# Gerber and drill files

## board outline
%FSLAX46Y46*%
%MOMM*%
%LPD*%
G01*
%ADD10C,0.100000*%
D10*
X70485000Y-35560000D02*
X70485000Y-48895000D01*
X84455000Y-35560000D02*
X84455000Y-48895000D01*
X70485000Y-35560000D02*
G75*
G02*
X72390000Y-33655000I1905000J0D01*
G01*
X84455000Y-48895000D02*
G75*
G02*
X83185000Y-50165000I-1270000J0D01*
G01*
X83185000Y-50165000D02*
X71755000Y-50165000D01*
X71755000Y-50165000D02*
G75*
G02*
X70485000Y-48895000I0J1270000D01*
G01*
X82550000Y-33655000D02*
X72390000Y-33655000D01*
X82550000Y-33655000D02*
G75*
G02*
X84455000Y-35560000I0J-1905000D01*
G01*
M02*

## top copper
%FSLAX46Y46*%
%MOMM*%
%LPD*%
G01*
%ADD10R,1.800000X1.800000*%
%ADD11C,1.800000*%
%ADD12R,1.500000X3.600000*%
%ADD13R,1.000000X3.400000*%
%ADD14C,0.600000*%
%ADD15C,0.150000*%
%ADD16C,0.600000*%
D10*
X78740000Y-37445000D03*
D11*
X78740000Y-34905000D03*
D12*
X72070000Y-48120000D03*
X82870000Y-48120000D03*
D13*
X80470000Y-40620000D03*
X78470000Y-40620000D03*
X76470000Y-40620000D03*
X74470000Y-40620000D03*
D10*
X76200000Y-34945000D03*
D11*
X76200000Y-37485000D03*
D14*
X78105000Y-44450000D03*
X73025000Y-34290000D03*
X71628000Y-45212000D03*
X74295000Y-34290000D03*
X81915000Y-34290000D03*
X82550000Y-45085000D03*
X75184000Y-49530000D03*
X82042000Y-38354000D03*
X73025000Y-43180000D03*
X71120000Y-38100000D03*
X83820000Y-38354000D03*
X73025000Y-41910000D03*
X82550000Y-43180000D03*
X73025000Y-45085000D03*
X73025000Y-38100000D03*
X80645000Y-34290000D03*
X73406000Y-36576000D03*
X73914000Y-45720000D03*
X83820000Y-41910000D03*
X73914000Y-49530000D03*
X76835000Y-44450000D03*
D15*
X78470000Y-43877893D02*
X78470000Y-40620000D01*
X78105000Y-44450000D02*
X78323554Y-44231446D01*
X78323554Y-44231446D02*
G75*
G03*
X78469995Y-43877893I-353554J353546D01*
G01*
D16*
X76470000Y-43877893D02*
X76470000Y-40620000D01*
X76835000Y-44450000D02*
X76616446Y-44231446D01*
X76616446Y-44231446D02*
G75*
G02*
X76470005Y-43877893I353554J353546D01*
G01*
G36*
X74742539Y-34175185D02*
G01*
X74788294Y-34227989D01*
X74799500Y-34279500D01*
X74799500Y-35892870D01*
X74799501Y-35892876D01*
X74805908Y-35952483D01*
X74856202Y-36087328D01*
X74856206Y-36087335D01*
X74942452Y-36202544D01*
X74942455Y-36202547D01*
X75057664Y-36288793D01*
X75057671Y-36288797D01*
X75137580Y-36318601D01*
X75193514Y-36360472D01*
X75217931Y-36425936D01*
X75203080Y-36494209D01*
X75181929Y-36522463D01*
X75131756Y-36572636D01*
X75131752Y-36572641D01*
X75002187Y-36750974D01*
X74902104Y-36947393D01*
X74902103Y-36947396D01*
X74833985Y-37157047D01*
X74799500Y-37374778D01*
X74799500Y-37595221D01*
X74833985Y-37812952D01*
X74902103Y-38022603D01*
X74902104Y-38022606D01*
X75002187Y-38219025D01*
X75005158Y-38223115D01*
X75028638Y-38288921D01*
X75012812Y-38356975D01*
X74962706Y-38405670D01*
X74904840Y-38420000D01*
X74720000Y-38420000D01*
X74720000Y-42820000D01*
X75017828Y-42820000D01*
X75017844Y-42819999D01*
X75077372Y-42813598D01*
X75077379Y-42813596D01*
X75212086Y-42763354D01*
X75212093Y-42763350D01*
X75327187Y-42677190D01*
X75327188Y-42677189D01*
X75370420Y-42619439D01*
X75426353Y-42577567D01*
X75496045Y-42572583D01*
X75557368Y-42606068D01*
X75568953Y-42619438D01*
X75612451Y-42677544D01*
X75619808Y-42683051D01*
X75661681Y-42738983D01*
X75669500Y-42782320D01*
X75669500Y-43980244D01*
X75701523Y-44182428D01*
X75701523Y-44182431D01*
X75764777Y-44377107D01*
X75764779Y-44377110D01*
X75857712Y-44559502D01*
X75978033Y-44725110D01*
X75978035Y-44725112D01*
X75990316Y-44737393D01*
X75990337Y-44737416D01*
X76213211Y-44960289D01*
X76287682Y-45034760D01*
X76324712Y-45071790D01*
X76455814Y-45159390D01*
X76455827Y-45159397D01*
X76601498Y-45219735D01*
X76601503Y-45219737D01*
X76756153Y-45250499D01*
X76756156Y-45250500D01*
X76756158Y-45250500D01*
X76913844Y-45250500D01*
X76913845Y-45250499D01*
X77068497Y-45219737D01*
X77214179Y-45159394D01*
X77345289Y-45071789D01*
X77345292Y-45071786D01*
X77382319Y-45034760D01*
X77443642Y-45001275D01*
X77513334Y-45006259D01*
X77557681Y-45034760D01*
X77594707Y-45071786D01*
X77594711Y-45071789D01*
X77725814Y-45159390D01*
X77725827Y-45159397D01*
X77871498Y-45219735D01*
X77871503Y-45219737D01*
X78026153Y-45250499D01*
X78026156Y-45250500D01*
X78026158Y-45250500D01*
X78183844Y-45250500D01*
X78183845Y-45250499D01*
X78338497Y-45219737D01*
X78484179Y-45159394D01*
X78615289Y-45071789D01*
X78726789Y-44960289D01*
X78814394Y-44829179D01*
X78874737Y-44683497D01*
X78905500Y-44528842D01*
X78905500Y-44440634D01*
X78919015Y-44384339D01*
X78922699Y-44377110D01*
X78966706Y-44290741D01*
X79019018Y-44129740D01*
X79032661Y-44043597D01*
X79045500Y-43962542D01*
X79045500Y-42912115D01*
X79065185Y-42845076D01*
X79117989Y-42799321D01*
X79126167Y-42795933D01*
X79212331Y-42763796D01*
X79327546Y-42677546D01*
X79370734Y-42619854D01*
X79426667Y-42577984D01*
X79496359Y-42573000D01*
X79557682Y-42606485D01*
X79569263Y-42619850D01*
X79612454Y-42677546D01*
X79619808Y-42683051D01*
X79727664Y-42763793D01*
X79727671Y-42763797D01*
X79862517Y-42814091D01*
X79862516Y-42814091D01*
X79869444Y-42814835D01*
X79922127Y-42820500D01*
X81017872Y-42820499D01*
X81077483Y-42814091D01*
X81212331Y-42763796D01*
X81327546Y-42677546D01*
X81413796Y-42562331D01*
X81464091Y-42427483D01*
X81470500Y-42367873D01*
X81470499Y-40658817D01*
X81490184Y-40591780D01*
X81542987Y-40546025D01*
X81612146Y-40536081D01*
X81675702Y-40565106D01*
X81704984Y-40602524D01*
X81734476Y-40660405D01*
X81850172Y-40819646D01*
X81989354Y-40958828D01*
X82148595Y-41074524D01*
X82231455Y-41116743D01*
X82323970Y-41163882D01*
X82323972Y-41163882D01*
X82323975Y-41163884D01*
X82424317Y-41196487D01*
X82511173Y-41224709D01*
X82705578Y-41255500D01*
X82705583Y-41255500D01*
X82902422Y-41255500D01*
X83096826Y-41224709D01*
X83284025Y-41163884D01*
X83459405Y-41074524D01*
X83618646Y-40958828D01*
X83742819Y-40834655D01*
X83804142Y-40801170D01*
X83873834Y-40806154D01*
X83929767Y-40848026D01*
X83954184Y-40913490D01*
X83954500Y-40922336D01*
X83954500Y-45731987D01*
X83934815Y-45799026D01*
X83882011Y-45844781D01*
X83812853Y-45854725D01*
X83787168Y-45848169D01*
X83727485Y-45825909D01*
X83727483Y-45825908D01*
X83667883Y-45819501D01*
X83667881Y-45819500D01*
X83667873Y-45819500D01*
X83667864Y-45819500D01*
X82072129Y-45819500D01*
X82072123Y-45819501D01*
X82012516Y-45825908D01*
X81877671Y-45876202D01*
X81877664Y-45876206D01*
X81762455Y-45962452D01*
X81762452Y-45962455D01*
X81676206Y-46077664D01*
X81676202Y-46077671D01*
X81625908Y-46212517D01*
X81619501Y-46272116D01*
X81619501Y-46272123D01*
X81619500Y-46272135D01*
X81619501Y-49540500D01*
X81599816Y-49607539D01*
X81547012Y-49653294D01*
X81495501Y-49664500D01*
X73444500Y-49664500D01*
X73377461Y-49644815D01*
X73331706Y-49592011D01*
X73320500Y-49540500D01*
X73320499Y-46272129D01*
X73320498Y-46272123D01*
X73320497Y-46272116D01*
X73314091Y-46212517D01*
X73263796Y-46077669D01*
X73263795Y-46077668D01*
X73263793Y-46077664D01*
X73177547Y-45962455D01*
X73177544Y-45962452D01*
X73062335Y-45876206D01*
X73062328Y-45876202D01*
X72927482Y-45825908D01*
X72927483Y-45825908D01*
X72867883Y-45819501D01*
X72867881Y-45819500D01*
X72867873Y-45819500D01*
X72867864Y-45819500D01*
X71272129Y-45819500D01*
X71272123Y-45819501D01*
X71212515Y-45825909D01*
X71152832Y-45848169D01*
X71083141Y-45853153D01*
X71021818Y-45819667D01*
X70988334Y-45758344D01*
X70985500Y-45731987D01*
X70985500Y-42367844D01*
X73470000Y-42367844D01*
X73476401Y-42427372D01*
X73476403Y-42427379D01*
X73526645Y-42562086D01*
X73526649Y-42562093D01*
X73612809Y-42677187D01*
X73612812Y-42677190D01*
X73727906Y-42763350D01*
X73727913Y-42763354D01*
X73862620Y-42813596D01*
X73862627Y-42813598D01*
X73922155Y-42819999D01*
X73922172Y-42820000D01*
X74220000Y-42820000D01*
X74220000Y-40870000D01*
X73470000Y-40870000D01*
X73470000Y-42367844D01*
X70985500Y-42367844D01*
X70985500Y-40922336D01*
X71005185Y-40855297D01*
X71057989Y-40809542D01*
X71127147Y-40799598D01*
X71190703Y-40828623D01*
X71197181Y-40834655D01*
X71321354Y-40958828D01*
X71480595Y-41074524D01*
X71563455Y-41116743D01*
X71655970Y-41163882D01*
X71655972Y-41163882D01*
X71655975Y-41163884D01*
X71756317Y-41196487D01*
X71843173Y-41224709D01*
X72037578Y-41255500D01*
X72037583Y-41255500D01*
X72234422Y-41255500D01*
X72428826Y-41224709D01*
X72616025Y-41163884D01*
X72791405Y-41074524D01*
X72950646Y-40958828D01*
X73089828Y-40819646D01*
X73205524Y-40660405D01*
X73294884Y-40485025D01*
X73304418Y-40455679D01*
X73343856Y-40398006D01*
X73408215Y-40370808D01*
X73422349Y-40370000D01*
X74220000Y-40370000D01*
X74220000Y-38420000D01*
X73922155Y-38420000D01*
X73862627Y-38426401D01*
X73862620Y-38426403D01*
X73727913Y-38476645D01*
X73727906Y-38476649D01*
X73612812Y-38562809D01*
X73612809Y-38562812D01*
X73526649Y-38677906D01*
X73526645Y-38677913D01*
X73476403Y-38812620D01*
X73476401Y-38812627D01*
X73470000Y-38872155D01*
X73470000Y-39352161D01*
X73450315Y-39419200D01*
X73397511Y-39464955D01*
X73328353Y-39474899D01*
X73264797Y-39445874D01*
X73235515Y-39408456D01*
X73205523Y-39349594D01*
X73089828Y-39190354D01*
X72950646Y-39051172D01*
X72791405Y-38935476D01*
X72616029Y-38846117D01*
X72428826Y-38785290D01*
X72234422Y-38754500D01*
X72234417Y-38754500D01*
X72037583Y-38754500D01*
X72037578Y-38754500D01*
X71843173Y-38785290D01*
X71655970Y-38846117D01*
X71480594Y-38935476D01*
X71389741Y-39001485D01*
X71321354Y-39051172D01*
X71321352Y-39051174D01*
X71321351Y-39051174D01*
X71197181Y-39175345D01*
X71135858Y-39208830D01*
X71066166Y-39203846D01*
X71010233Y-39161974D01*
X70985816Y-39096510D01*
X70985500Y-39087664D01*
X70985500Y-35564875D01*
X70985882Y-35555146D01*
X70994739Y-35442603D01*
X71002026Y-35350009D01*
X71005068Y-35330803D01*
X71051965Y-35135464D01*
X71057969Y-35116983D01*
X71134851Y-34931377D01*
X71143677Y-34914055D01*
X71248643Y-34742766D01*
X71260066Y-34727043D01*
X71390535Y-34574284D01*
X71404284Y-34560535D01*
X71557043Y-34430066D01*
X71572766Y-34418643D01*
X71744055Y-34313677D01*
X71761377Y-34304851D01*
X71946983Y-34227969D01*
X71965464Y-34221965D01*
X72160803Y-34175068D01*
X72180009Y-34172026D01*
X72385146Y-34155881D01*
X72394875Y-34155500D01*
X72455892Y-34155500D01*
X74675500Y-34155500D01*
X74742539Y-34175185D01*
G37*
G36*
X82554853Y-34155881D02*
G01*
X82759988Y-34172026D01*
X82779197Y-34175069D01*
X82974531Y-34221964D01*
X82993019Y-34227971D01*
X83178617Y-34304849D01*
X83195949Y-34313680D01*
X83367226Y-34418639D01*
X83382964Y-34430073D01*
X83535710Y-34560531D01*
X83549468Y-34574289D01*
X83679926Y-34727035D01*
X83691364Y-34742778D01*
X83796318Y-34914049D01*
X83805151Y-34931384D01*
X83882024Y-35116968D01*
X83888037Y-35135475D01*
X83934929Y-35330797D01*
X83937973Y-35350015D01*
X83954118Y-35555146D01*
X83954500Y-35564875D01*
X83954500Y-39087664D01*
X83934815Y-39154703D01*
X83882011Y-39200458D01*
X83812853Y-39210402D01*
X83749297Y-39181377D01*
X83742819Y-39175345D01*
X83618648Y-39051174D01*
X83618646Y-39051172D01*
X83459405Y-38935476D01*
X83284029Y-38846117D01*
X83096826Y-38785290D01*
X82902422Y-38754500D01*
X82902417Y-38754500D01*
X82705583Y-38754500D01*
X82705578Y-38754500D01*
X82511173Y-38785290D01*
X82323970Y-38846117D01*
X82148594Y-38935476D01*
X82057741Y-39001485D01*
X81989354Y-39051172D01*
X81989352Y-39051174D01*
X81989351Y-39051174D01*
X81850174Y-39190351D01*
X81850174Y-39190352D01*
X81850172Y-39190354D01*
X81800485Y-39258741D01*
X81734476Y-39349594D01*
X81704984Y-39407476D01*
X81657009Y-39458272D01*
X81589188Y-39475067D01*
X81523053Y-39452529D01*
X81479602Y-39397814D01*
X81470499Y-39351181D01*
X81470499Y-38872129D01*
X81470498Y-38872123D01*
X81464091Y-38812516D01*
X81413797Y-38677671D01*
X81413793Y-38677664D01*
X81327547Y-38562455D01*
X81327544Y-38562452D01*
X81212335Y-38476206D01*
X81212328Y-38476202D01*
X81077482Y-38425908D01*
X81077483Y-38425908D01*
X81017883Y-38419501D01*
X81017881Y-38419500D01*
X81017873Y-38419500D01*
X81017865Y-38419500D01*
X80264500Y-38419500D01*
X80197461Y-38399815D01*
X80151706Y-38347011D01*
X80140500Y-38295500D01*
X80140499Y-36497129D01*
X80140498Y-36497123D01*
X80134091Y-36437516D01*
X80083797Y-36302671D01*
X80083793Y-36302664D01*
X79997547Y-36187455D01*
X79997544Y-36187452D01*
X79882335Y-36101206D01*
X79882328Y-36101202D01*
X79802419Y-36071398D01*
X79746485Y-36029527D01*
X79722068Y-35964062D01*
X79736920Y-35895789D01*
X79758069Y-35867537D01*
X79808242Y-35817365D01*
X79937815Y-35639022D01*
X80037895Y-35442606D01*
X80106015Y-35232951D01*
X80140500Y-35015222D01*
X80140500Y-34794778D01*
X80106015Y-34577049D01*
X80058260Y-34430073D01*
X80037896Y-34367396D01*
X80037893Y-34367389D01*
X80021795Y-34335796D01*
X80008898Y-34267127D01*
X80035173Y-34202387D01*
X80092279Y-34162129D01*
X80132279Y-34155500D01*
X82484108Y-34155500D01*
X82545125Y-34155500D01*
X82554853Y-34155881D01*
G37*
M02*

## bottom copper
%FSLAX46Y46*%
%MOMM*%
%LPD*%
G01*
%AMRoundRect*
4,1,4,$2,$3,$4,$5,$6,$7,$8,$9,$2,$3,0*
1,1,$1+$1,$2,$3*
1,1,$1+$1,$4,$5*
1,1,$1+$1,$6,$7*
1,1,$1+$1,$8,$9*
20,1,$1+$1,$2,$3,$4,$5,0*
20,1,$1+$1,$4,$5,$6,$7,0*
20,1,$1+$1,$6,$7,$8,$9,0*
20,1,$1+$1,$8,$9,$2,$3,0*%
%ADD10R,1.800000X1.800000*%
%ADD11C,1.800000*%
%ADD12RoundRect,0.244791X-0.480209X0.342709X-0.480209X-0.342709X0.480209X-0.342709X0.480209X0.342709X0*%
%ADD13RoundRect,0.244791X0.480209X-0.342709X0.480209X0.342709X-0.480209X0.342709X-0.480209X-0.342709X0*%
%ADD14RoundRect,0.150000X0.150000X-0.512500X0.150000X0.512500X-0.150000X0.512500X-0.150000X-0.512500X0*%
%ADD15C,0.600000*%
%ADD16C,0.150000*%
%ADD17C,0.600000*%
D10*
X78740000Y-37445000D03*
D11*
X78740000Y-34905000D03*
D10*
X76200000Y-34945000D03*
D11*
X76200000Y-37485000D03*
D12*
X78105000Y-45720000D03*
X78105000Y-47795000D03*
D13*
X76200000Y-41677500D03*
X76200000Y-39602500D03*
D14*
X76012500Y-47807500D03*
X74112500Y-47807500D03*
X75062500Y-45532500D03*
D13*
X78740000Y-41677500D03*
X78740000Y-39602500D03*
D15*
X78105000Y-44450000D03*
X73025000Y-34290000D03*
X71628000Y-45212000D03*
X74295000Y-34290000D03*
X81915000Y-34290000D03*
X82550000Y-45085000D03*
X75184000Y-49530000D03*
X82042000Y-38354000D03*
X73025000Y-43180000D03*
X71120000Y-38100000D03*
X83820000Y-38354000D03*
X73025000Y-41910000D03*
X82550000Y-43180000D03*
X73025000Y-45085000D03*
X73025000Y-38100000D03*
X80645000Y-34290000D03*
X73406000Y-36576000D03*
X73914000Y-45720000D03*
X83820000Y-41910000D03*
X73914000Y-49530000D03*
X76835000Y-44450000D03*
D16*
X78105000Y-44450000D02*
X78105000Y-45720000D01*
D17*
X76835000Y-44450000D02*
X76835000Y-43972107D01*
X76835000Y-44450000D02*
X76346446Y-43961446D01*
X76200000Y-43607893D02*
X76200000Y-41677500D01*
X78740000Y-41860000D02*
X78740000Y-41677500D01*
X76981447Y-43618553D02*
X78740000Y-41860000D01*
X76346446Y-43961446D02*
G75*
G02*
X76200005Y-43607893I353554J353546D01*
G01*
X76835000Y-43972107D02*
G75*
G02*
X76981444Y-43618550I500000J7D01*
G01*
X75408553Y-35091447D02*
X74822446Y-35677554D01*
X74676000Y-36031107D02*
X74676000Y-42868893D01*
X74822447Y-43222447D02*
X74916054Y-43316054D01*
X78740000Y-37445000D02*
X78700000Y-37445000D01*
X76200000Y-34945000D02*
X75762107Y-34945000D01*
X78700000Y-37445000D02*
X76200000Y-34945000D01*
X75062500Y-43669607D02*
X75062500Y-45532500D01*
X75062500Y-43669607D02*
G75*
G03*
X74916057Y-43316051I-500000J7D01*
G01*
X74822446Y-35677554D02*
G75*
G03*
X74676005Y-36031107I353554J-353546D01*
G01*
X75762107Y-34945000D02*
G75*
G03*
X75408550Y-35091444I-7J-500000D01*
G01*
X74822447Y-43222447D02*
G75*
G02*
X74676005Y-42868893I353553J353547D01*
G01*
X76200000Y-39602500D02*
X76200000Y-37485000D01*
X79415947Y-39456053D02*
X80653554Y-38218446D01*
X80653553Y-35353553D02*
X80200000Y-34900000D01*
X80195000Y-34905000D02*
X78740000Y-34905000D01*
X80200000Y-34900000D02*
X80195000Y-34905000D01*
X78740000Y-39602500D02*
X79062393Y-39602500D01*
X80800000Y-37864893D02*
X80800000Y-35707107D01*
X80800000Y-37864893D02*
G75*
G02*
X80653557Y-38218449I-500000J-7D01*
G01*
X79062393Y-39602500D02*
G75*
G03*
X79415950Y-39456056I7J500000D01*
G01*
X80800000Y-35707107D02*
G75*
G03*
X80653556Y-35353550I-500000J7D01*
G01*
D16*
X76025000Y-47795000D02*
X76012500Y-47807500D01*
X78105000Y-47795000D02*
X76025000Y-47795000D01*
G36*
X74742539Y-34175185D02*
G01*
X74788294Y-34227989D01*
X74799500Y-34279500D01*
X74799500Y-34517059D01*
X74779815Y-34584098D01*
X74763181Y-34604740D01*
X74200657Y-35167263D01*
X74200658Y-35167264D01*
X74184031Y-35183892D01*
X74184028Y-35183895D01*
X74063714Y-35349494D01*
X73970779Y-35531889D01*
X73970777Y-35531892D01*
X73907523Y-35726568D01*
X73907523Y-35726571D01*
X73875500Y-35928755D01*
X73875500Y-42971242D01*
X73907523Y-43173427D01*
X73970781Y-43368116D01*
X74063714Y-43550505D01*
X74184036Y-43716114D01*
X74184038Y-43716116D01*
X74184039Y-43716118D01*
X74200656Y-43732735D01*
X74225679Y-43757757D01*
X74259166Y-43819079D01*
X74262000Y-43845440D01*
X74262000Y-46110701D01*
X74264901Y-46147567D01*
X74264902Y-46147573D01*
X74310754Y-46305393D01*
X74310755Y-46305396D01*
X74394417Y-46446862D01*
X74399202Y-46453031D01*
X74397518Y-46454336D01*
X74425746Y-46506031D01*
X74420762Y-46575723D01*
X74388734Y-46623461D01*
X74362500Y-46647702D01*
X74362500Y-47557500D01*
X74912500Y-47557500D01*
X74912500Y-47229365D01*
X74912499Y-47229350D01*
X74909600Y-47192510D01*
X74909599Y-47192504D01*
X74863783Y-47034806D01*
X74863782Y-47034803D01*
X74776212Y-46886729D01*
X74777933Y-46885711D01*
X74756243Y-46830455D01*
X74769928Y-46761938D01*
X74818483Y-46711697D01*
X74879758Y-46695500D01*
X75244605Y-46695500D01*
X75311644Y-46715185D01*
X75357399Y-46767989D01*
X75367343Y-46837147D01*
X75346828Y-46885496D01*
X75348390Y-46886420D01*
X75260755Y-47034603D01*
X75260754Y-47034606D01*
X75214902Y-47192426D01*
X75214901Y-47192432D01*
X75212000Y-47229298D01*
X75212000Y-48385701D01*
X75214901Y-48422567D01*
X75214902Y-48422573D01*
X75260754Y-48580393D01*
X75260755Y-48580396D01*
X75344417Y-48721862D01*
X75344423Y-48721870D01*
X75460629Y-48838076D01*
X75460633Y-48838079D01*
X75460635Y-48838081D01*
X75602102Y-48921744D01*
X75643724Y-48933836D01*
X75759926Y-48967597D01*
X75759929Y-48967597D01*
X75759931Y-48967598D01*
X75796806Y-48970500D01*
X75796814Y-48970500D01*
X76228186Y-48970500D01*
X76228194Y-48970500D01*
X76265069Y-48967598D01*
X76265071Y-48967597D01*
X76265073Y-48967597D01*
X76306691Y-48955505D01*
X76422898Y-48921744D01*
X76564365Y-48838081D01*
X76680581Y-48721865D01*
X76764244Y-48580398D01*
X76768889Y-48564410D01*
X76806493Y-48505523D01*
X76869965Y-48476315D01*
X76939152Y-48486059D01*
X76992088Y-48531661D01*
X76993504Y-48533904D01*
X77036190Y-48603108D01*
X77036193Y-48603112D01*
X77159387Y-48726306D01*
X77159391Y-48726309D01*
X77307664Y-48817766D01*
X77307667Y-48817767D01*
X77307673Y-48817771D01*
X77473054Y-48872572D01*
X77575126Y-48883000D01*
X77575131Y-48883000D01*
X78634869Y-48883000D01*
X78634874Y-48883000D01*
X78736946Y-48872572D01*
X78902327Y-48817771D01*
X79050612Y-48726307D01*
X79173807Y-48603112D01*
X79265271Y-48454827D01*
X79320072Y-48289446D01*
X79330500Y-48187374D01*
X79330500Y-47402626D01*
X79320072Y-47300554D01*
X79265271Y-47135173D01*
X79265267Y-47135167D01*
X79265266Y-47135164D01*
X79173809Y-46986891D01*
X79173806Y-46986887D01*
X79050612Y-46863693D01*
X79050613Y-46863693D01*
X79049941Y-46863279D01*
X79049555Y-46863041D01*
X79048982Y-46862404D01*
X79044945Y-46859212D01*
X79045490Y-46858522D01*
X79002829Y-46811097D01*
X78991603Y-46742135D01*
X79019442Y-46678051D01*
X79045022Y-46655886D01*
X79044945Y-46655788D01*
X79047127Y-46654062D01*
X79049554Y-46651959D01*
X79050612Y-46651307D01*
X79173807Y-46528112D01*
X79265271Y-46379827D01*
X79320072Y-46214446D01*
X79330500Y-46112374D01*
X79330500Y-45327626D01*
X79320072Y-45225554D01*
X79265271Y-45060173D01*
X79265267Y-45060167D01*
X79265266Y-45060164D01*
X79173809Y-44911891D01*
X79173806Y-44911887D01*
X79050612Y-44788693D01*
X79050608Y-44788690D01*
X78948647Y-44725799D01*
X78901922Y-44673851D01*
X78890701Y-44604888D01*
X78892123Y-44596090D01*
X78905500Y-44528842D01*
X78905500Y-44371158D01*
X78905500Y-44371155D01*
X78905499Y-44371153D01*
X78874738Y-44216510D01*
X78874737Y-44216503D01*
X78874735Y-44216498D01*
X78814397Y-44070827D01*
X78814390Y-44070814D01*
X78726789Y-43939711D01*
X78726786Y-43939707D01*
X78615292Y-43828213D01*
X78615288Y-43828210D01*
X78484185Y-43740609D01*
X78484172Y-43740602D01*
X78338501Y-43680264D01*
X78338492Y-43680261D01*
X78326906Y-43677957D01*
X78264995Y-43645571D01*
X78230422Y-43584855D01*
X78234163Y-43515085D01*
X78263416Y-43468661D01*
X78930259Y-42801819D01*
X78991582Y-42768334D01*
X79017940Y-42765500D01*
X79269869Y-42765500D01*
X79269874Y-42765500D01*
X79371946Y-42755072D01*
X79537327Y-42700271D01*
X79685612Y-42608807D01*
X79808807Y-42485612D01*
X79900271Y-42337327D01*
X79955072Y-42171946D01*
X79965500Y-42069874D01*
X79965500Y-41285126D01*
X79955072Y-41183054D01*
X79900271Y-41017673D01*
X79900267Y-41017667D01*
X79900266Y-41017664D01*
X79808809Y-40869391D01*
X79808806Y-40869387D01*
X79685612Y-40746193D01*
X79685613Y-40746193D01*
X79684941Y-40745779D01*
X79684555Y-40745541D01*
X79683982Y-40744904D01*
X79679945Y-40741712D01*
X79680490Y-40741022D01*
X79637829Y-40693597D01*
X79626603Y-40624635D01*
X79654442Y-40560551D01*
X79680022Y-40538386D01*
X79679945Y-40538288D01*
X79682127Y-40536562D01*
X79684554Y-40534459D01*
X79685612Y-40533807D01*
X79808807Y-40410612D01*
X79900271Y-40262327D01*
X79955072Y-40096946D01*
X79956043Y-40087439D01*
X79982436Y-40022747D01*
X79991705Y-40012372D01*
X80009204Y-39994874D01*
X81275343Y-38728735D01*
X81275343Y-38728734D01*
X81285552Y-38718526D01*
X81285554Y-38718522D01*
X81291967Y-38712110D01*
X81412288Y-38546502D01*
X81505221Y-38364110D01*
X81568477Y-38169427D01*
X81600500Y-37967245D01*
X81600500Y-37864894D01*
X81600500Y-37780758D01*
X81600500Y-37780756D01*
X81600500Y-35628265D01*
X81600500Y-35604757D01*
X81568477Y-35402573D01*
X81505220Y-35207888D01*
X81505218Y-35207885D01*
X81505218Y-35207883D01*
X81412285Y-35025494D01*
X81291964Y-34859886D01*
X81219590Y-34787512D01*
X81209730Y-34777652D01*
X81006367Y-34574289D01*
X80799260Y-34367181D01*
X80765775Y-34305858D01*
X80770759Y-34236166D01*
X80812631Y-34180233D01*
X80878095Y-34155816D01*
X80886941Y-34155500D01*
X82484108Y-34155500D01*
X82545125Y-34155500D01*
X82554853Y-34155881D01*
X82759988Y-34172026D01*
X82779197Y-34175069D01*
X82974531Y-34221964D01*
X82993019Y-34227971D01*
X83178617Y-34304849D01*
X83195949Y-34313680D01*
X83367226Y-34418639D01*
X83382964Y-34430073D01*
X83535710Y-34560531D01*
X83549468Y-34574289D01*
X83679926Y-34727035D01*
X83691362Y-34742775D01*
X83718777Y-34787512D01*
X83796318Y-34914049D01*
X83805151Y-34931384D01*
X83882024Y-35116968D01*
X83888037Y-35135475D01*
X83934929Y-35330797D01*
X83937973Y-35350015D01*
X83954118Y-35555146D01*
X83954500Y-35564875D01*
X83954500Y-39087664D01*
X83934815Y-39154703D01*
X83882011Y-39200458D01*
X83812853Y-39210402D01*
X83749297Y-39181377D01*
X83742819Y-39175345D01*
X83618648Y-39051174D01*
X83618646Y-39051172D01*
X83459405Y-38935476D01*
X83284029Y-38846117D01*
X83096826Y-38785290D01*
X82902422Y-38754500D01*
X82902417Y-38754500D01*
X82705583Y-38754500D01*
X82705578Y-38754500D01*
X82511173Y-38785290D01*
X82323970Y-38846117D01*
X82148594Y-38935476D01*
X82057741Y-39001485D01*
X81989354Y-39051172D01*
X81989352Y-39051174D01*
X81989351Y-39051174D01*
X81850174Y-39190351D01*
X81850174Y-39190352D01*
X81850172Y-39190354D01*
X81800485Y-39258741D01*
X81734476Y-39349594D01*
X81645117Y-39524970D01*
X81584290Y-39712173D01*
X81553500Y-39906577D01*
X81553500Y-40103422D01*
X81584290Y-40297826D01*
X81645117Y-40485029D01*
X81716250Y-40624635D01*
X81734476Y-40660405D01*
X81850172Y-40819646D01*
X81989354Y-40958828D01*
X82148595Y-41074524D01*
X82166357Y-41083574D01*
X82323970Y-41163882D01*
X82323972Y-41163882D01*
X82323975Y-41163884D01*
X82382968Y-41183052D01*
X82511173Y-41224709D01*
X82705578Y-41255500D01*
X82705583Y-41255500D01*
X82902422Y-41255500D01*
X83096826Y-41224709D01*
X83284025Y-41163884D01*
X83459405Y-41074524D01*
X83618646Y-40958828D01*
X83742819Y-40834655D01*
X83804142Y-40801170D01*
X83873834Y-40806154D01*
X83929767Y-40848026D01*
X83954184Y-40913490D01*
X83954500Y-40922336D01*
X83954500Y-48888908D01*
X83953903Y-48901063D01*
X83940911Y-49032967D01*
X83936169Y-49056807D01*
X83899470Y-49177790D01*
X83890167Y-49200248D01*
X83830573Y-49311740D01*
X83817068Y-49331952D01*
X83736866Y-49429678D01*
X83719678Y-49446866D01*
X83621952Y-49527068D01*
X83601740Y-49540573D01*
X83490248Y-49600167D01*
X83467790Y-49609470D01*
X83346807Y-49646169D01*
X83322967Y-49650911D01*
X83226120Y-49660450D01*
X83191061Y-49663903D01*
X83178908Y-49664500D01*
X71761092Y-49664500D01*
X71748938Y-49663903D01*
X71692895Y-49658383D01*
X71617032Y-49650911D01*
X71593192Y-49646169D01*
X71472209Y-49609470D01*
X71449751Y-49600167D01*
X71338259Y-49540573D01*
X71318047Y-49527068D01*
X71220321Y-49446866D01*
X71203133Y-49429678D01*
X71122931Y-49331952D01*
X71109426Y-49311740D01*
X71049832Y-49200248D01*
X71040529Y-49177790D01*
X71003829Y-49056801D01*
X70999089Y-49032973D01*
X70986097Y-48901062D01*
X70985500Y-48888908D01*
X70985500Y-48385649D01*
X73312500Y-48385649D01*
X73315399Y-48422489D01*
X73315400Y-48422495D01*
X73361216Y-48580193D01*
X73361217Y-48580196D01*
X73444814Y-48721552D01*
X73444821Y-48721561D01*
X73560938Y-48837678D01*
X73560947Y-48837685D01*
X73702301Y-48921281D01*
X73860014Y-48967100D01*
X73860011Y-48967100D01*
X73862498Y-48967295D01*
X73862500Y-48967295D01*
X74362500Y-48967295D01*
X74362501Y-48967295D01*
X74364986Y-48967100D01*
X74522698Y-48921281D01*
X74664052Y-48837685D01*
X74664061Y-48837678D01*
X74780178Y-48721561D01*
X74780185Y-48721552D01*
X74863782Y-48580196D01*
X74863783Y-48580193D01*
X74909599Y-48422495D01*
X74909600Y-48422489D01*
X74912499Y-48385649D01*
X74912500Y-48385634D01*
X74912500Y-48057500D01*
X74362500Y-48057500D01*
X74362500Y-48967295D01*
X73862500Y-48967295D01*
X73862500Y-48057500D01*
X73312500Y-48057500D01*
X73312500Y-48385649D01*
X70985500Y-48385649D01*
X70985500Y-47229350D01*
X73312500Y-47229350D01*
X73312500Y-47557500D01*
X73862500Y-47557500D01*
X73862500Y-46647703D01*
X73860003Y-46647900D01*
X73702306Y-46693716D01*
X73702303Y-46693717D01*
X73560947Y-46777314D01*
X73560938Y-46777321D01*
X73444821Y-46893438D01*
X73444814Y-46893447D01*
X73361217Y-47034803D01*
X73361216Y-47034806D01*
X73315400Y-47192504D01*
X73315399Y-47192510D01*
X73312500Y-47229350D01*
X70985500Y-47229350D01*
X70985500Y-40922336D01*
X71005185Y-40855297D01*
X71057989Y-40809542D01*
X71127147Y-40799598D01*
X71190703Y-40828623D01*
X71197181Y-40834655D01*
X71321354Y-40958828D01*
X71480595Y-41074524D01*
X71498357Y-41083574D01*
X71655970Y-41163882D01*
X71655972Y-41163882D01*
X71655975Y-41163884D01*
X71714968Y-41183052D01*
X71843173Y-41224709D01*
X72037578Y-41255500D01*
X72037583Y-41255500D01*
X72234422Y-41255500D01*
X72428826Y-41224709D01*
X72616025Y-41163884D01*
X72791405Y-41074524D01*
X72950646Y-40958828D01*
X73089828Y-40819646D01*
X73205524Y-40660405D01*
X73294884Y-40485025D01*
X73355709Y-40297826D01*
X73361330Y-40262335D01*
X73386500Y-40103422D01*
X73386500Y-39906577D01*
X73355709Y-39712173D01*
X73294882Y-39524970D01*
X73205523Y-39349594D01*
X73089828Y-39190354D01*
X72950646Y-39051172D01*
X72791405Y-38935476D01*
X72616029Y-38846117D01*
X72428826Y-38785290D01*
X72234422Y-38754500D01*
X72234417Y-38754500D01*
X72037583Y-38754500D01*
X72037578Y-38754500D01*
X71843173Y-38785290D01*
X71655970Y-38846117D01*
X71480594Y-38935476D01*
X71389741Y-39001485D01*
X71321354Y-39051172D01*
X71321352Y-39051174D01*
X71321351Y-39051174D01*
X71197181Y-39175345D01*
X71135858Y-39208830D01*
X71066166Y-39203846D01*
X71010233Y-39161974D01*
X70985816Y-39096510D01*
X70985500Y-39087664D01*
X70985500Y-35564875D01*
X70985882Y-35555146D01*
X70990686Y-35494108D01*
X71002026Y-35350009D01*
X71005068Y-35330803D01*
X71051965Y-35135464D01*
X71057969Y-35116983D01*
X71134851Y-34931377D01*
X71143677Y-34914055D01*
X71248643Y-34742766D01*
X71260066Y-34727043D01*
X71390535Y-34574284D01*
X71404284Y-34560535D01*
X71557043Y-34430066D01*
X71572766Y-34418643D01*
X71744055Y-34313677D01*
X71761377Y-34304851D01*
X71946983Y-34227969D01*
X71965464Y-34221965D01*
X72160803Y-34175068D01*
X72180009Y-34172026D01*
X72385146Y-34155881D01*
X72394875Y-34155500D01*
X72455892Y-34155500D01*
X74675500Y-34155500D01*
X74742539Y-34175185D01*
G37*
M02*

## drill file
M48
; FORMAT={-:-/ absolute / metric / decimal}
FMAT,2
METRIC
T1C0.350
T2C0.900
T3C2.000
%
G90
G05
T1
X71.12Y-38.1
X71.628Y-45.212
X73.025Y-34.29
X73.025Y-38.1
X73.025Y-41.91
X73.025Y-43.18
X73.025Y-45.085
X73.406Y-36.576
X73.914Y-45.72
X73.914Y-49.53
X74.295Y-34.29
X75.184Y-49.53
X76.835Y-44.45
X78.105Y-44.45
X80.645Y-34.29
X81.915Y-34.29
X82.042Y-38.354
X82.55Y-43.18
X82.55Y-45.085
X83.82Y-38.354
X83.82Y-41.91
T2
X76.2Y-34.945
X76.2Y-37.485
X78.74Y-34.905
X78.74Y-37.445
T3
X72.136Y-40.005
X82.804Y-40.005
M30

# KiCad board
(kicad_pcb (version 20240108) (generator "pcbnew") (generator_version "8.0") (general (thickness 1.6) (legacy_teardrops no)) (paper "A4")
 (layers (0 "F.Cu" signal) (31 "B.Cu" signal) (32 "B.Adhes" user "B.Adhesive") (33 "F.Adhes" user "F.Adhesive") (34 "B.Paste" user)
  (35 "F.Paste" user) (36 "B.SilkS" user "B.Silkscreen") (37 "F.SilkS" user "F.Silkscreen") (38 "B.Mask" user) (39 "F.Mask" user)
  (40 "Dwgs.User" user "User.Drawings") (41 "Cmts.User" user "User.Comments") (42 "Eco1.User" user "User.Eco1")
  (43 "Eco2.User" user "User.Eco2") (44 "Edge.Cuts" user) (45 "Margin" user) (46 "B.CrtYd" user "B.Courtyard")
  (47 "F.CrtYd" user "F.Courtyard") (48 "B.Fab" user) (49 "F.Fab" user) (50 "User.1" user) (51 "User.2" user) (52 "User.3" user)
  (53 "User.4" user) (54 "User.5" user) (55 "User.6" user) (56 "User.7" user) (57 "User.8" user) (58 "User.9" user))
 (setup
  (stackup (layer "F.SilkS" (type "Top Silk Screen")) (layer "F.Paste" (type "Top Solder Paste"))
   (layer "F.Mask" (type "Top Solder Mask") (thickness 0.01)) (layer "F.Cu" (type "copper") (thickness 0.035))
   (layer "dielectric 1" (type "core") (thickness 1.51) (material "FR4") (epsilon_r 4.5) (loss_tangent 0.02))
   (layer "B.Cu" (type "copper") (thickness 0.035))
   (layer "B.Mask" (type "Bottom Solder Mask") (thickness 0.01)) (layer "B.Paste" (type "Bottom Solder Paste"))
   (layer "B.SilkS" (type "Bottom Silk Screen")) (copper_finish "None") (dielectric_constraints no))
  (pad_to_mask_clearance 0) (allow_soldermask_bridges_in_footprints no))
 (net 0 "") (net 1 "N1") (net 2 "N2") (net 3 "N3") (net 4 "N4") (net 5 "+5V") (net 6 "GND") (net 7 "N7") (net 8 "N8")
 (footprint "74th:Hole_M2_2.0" (layer "F.Cu") (at 72.136 40.005)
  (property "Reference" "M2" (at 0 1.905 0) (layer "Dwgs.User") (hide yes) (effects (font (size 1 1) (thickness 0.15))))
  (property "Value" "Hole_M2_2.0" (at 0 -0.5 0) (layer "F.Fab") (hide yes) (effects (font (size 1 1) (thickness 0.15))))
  (pad "" np_thru_hole circle (at 0 0) (size 2 2) (drill 2) (layers "F&B.Cu" "*.Mask")))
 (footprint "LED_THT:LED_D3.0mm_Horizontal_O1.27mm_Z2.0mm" (layer "F.Cu") (at 78.74 37.445 90)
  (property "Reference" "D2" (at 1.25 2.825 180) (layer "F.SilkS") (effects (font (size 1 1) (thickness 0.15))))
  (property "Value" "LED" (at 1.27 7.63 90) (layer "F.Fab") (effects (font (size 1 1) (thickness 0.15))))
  (pad "1" thru_hole rect (at 0 0 90) (size 1.8 1.8) (drill 0.9) (layers "*.Cu" "*.Mask") (remove_unused_layers no) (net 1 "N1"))
  (pad "2" thru_hole circle (at 2.54 0 90) (size 1.8 1.8) (drill 0.9) (layers "*.Cu" "*.Mask") (remove_unused_layers no) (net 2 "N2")))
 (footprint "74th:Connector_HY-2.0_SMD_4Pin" (layer "F.Cu") (at 77.47 40.62)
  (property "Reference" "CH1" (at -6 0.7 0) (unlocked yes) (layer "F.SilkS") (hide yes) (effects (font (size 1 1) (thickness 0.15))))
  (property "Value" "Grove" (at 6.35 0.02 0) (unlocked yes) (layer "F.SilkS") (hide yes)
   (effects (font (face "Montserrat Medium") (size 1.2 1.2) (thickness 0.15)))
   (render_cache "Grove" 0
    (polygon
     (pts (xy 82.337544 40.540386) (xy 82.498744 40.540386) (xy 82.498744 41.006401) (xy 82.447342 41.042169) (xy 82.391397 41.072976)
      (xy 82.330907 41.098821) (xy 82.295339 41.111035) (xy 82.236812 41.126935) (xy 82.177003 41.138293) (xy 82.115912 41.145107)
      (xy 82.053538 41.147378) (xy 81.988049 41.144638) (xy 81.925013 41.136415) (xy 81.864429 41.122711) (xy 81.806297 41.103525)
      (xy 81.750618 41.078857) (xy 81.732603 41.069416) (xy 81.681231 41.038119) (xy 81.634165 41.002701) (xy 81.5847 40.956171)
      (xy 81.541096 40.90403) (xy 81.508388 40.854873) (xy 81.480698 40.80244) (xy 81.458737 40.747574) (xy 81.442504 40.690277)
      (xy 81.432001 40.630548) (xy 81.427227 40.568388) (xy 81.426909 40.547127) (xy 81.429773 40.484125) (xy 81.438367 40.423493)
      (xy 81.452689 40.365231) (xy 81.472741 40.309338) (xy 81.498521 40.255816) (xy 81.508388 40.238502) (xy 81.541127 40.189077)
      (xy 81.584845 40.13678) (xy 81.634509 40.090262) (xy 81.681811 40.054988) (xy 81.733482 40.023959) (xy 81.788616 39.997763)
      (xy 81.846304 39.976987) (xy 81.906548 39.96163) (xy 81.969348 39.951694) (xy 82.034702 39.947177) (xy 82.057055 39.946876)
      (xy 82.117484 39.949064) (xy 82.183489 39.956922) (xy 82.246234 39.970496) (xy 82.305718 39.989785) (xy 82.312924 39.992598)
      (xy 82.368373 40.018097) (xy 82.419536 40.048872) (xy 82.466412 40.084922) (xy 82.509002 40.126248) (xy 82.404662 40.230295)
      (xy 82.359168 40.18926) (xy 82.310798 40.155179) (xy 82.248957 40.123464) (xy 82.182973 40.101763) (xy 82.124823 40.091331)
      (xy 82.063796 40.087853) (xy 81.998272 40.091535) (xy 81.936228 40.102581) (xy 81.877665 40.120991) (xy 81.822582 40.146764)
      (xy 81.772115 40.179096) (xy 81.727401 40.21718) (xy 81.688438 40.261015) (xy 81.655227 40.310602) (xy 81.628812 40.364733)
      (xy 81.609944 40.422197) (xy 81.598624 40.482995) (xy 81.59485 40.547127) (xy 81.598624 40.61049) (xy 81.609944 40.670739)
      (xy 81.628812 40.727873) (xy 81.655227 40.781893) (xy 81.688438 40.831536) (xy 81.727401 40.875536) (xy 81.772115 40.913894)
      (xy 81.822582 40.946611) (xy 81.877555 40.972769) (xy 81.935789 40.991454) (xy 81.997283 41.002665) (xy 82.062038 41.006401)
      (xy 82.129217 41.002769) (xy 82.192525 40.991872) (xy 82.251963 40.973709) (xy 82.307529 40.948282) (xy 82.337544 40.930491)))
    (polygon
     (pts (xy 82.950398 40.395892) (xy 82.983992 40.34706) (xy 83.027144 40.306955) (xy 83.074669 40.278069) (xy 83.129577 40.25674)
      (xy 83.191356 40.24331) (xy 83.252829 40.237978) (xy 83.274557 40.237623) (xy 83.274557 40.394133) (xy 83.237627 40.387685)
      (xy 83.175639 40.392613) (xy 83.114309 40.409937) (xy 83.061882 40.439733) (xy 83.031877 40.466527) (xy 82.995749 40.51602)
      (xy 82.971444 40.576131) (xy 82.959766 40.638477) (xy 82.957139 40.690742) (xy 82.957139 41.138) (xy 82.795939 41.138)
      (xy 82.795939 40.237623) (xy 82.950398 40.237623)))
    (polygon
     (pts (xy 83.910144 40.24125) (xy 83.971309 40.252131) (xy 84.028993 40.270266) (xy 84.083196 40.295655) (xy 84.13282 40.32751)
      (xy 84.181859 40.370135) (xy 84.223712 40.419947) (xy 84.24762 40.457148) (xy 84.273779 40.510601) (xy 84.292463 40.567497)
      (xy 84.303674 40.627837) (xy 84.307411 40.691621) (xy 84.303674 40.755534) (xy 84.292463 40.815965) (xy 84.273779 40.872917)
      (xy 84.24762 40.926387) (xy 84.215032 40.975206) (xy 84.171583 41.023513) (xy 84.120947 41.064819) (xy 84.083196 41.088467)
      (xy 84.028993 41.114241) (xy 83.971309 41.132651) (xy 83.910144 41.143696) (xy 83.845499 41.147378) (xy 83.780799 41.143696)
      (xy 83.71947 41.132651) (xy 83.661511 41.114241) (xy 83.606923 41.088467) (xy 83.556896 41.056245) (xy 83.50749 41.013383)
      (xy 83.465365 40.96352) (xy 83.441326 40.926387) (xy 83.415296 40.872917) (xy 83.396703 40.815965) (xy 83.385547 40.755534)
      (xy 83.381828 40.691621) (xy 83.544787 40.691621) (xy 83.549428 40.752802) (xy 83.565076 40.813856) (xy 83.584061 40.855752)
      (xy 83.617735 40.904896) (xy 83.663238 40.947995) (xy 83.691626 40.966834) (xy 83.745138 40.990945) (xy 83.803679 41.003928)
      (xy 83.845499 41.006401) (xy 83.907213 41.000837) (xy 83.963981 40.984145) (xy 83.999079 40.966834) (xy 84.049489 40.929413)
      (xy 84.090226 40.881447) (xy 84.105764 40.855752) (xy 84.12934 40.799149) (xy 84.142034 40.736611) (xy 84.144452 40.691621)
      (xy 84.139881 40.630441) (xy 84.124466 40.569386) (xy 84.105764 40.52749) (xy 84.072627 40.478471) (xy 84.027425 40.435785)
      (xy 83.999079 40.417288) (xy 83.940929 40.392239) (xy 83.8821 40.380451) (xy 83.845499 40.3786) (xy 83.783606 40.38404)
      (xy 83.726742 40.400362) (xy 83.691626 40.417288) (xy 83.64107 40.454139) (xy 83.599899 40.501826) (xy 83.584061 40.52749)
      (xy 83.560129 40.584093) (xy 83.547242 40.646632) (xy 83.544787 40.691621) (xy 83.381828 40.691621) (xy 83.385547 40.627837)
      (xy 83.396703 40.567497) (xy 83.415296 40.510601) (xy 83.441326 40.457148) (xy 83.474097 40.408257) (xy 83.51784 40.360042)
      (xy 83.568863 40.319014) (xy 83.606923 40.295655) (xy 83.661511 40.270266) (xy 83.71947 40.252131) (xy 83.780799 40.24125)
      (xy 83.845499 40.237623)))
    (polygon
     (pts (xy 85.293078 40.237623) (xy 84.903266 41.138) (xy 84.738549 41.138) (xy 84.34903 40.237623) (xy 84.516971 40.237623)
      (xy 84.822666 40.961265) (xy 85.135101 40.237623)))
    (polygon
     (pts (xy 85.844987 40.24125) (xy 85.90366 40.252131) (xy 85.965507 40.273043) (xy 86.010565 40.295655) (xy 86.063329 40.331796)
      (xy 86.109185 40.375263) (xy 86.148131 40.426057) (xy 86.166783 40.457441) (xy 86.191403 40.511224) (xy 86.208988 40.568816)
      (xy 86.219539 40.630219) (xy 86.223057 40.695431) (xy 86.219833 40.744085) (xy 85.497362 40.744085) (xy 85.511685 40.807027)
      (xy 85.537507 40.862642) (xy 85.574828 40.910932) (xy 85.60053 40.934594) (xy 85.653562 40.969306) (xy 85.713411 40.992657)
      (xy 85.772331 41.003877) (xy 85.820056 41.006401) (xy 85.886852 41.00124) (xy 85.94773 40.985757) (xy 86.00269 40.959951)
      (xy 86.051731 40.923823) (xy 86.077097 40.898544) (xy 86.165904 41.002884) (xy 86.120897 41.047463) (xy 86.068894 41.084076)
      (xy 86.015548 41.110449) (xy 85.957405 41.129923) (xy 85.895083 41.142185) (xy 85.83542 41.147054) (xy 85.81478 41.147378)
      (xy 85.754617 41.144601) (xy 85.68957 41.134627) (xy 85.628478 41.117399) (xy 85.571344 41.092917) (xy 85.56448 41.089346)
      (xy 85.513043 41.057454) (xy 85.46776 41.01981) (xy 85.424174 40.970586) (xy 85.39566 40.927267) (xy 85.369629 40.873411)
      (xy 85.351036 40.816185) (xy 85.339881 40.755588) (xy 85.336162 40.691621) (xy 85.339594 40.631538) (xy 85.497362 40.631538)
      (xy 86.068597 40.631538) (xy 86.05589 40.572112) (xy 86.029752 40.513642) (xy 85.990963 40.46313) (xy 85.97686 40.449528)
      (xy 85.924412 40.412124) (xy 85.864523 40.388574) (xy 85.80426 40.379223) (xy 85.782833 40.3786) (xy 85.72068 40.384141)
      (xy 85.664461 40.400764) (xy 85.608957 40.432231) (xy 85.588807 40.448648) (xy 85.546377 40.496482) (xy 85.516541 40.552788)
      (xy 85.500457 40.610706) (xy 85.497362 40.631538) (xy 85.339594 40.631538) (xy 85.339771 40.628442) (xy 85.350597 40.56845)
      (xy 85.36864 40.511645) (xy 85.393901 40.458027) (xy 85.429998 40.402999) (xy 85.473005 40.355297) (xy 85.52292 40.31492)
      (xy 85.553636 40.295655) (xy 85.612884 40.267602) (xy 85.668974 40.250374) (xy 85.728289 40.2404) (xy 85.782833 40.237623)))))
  (pad "" smd rect (at -5.4 7.5 180) (size 1.5 3.6) (layers "F.Cu" "F.Paste" "F.Mask"))
  (pad "" smd rect (at 5.4 7.5 180) (size 1.5 3.6) (layers "F.Cu" "F.Paste" "F.Mask"))
  (pad "1" smd rect (at 3 0 180) (size 1 3.4) (layers "F.Cu" "F.Paste" "F.Mask") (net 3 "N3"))
  (pad "2" smd rect (at 1 0 180) (size 1 3.4) (layers "F.Cu" "F.Paste" "F.Mask") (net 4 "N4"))
  (pad "3" smd rect (at -1 0 180) (size 1 3.4) (layers "F.Cu" "F.Paste" "F.Mask") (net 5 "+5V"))
  (pad "4" smd rect (at -3 0 180) (size 1 3.4) (layers "F.Cu" "F.Paste" "F.Mask") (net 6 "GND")))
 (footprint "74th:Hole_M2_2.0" (layer "F.Cu") (at 82.804 40.005)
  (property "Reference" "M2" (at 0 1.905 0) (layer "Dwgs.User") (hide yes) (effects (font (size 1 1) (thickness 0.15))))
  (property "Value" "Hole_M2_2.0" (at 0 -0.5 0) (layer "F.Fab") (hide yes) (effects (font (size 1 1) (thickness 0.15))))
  (pad "" np_thru_hole circle (at 0 0) (size 2 2) (drill 2) (layers "F&B.Cu" "*.Mask")))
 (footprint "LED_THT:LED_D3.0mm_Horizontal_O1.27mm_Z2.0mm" (layer "F.Cu") (at 76.2 34.945 -90)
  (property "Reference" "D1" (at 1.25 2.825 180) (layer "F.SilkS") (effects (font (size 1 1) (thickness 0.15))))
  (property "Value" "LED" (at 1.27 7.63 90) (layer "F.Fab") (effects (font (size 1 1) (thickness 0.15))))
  (pad "1" thru_hole rect (at 0 0 270) (size 1.8 1.8) (drill 0.9) (layers "*.Cu" "*.Mask") (remove_unused_layers no) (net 1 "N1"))
  (pad "2" thru_hole circle (at 2.54 0 270) (size 1.8 1.8) (drill 0.9) (layers "*.Cu" "*.Mask") (remove_unused_layers no) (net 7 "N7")))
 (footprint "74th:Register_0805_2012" (layer "B.Cu") (at 78.105 46.7575 -90)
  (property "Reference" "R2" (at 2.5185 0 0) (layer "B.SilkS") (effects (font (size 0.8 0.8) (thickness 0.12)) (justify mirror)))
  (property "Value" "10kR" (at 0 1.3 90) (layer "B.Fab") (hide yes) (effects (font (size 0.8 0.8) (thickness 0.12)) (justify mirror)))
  (pad "1" smd roundrect (at -1.0375 0 270) (size 1.175 1.45) (layers "B.Cu" "B.Paste" "B.Mask") (roundrect_rratio 0.208333) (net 4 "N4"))
  (pad "2" smd roundrect (at 1.0375 0 270) (size 1.175 1.45) (layers "B.Cu" "B.Paste" "B.Mask") (roundrect_rratio 0.208333) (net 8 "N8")))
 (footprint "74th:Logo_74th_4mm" (layer "B.Cu") (at 72.644 36.576 90)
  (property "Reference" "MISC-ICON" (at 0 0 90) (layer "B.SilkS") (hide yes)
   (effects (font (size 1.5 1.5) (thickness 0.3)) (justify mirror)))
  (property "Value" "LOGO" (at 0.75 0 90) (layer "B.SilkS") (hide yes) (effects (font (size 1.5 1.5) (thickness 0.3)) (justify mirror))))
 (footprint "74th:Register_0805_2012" (layer "B.Cu") (at 76.2 40.64 90)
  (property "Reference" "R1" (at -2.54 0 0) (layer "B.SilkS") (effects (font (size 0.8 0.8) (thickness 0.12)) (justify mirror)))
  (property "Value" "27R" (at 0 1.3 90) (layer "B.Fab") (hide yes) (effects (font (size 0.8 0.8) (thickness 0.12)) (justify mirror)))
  (pad "1" smd roundrect (at -1.0375 0 90) (size 1.175 1.45) (layers "B.Cu" "B.Paste" "B.Mask") (roundrect_rratio 0.208333) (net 5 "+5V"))
  (pad "2" smd roundrect (at 1.0375 0 90) (size 1.175 1.45) (layers "B.Cu" "B.Paste" "B.Mask") (roundrect_rratio 0.208333) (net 7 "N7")))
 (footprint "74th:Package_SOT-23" (layer "B.Cu") (at 75.0625 46.67 90)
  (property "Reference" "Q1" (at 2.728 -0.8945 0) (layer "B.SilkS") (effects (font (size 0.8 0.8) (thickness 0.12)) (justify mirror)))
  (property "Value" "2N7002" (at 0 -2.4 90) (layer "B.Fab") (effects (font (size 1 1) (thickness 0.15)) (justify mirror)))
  (pad "1" smd roundrect (at -1.1375 0.95 90) (size 1.325 0.6) (layers "B.Cu" "B.Paste" "B.Mask") (roundrect_rratio 0.25) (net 8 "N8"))
  (pad "2" smd roundrect (at -1.1375 -0.95 90) (size 1.325 0.6) (layers "B.Cu" "B.Paste" "B.Mask") (roundrect_rratio 0.25) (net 6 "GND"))
  (pad "3" smd roundrect (at 1.1375 0 90) (size 1.325 0.6) (layers "B.Cu" "B.Paste" "B.Mask") (roundrect_rratio 0.25) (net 1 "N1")))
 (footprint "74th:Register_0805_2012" (layer "B.Cu") (at 78.74 40.64 90)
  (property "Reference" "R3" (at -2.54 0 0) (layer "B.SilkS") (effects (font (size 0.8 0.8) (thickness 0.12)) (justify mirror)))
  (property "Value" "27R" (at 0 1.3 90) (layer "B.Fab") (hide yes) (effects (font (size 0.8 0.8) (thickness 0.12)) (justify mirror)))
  (pad "1" smd roundrect (at -1.0375 0 90) (size 1.175 1.45) (layers "B.Cu" "B.Paste" "B.Mask") (roundrect_rratio 0.208333) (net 5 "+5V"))
  (pad "2" smd roundrect (at 1.0375 0 90) (size 1.175 1.45) (layers "B.Cu" "B.Paste" "B.Mask") (roundrect_rratio 0.208333) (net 2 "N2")))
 (gr_line (start 70.485 35.56) (end 70.485 48.895) (stroke (width 0.1) (type default)) (layer "Edge.Cuts"))
 (gr_line (start 84.455 35.56) (end 84.455 48.895) (stroke (width 0.1) (type default)) (layer "Edge.Cuts"))
 (gr_arc (start 70.485 35.56) (mid 71.042962 34.212962) (end 72.39 33.655) (stroke (width 0.1) (type default)) (layer "Edge.Cuts"))
 (gr_arc (start 84.455 48.895) (mid 84.083026 49.793026) (end 83.185 50.165) (stroke (width 0.1) (type default)) (layer "Edge.Cuts"))
 (gr_line (start 83.185 50.165) (end 71.755 50.165) (stroke (width 0.1) (type default)) (layer "Edge.Cuts"))
 (gr_arc (start 71.755 50.165) (mid 70.856974 49.793026) (end 70.485 48.895) (stroke (width 0.1) (type default)) (layer "Edge.Cuts"))
 (gr_line (start 82.55 33.655) (end 72.39 33.655) (stroke (width 0.1) (type default)) (layer "Edge.Cuts"))
 (gr_arc (start 82.55 33.655) (mid 83.897038 34.212962) (end 84.455 35.56) (stroke (width 0.1) (type default)) (layer "Edge.Cuts"))
 (segment (start 78.47 43.877893) (end 78.47 40.62) (width 0.15) (layer "F.Cu") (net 4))
 (segment (start 78.105 44.45) (end 78.323554 44.231446) (width 0.15) (layer "F.Cu") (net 4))
 (via (at 78.105 44.45) (size 0.6) (drill 0.35) (layers "F.Cu" "B.Cu") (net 4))
 (arc (start 78.323554 44.231446) (mid 78.43194 44.069234) (end 78.47 43.877893) (width 0.15) (layer "F.Cu") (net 4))
 (segment (start 78.105 44.45) (end 78.105 45.72) (width 0.15) (layer "B.Cu") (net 4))
 (via (at 73.025 34.29) (size 0.6) (drill 0.35) (layers "F.Cu" "B.Cu") (free yes) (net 6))
 (via (at 71.628 45.212) (size 0.6) (drill 0.35) (layers "F.Cu" "B.Cu") (free yes) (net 6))
 (via (at 74.295 34.29) (size 0.6) (drill 0.35) (layers "F.Cu" "B.Cu") (free yes) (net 6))
 (via (at 81.915 34.29) (size 0.6) (drill 0.35) (layers "F.Cu" "B.Cu") (free yes) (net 6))
 (via (at 82.55 45.085) (size 0.6) (drill 0.35) (layers "F.Cu" "B.Cu") (free yes) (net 6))
 (via (at 75.184 49.53) (size 0.6) (drill 0.35) (layers "F.Cu" "B.Cu") (free yes) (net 6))
 (via (at 82.042 38.354) (size 0.6) (drill 0.35) (layers "F.Cu" "B.Cu") (free yes) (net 6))
 (via (at 73.025 43.18) (size 0.6) (drill 0.35) (layers "F.Cu" "B.Cu") (free yes) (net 6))
 (via (at 71.12 38.1) (size 0.6) (drill 0.35) (layers "F.Cu" "B.Cu") (free yes) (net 6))
 (via (at 83.82 38.354) (size 0.6) (drill 0.35) (layers "F.Cu" "B.Cu") (free yes) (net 6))
 (via (at 73.025 41.91) (size 0.6) (drill 0.35) (layers "F.Cu" "B.Cu") (free yes) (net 6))
 (via (at 82.55 43.18) (size 0.6) (drill 0.35) (layers "F.Cu" "B.Cu") (free yes) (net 6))
 (via (at 73.025 45.085) (size 0.6) (drill 0.35) (layers "F.Cu" "B.Cu") (free yes) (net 6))
 (via (at 73.025 38.1) (size 0.6) (drill 0.35) (layers "F.Cu" "B.Cu") (free yes) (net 6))
 (via (at 80.645 34.29) (size 0.6) (drill 0.35) (layers "F.Cu" "B.Cu") (free yes) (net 6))
 (via (at 73.406 36.576) (size 0.6) (drill 0.35) (layers "F.Cu" "B.Cu") (free yes) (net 6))
 (via (at 73.914 45.72) (size 0.6) (drill 0.35) (layers "F.Cu" "B.Cu") (free yes) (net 6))
 (via (at 83.82 41.91) (size 0.6) (drill 0.35) (layers "F.Cu" "B.Cu") (free yes) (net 6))
 (via (at 73.914 49.53) (size 0.6) (drill 0.35) (layers "F.Cu" "B.Cu") (free yes) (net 6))
 (segment (start 76.47 43.877893) (end 76.47 40.62) (width 0.6) (layer "F.Cu") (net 5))
 (segment (start 76.835 44.45) (end 76.616446 44.231446) (width 0.6) (layer "F.Cu") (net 5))
 (via (at 76.835 44.45) (size 0.6) (drill 0.35) (layers "F.Cu" "B.Cu") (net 5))
 (arc (start 76.616446 44.231446) (mid 76.50806 44.069234) (end 76.47 43.877893) (width 0.6) (layer "F.Cu") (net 5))
 (segment (start 76.835 44.45) (end 76.835 43.972107) (width 0.6) (layer "B.Cu") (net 5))
 (segment (start 76.835 44.45) (end 76.346446 43.961446) (width 0.6) (layer "B.Cu") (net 5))
 (segment (start 76.2 43.607893) (end 76.2 41.6775) (width 0.6) (layer "B.Cu") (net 5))
 (segment (start 78.74 41.86) (end 78.74 41.6775) (width 0.6) (layer "B.Cu") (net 5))
 (segment (start 76.981447 43.618553) (end 78.74 41.86) (width 0.6) (layer "B.Cu") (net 5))
 (arc (start 76.346446 43.961446) (mid 76.23806 43.799234) (end 76.2 43.607893) (width 0.6) (layer "B.Cu") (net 5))
 (arc (start 76.835 43.972107) (mid 76.87306 43.780765) (end 76.981447 43.618553) (width 0.6) (layer "B.Cu") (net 5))
 (segment (start 75.408553 35.091447) (end 74.822446 35.677554) (width 0.6) (layer "B.Cu") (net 1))
 (segment (start 74.676 36.031107) (end 74.676 42.868893) (width 0.6) (layer "B.Cu") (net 1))
 (segment (start 74.822447 43.222447) (end 74.916054 43.316054) (width 0.6) (layer "B.Cu") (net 1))
 (segment (start 78.74 37.445) (end 78.7 37.445) (width 0.6) (layer "B.Cu") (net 1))
 (segment (start 76.2 34.945) (end 75.762107 34.945) (width 0.6) (layer "B.Cu") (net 1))
 (segment (start 78.7 37.445) (end 76.2 34.945) (width 0.6) (layer "B.Cu") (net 1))
 (segment (start 75.0625 43.669607) (end 75.0625 45.5325) (width 0.6) (layer "B.Cu") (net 1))
 (arc (start 75.0625 43.669607) (mid 75.02444 43.478266) (end 74.916054 43.316054) (width 0.6) (layer "B.Cu") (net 1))
 (arc (start 74.822446 35.677554) (mid 74.71406 35.839766) (end 74.676 36.031107) (width 0.6) (layer "B.Cu") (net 1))
 (arc (start 75.762107 34.945) (mid 75.570765 34.98306) (end 75.408553 35.091447) (width 0.6) (layer "B.Cu") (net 1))
 (arc (start 74.822447 43.222447) (mid 74.71406 43.060235) (end 74.676 42.868893) (width 0.6) (layer "B.Cu") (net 1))
 (segment (start 76.2 39.6025) (end 76.2 37.485) (width 0.6) (layer "B.Cu") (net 7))
 (segment (start 79.415947 39.456053) (end 80.653554 38.218446) (width 0.6) (layer "B.Cu") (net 2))
 (segment (start 80.653553 35.353553) (end 80.2 34.9) (width 0.6) (layer "B.Cu") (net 2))
 (segment (start 80.195 34.905) (end 78.74 34.905) (width 0.6) (layer "B.Cu") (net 2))
 (segment (start 80.2 34.9) (end 80.195 34.905) (width 0.6) (layer "B.Cu") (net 2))
 (segment (start 78.74 39.6025) (end 79.062393 39.6025) (width 0.6) (layer "B.Cu") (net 2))
 (segment (start 80.8 37.864893) (end 80.8 35.707107) (width 0.6) (layer "B.Cu") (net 2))
 (arc (start 80.8 37.864893) (mid 80.76194 38.056234) (end 80.653554 38.218446) (width 0.6) (layer "B.Cu") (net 2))
 (arc (start 79.062393 39.6025) (mid 79.253735 39.56444) (end 79.415947 39.456053) (width 0.6) (layer "B.Cu") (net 2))
 (arc (start 80.8 35.707107) (mid 80.76194 35.515765) (end 80.653553 35.353553) (width 0.6) (layer "B.Cu") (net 2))
 (segment (start 76.025 47.795) (end 76.0125 47.8075) (width 0.15) (layer "B.Cu") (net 8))
 (segment (start 78.105 47.795) (end 76.025 47.795) (width 0.15) (layer "B.Cu") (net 8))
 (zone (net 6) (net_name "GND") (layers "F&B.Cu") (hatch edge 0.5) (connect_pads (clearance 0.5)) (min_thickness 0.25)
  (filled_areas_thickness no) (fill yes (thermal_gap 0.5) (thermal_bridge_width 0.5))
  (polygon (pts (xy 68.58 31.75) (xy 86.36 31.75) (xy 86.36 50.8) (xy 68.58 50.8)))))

